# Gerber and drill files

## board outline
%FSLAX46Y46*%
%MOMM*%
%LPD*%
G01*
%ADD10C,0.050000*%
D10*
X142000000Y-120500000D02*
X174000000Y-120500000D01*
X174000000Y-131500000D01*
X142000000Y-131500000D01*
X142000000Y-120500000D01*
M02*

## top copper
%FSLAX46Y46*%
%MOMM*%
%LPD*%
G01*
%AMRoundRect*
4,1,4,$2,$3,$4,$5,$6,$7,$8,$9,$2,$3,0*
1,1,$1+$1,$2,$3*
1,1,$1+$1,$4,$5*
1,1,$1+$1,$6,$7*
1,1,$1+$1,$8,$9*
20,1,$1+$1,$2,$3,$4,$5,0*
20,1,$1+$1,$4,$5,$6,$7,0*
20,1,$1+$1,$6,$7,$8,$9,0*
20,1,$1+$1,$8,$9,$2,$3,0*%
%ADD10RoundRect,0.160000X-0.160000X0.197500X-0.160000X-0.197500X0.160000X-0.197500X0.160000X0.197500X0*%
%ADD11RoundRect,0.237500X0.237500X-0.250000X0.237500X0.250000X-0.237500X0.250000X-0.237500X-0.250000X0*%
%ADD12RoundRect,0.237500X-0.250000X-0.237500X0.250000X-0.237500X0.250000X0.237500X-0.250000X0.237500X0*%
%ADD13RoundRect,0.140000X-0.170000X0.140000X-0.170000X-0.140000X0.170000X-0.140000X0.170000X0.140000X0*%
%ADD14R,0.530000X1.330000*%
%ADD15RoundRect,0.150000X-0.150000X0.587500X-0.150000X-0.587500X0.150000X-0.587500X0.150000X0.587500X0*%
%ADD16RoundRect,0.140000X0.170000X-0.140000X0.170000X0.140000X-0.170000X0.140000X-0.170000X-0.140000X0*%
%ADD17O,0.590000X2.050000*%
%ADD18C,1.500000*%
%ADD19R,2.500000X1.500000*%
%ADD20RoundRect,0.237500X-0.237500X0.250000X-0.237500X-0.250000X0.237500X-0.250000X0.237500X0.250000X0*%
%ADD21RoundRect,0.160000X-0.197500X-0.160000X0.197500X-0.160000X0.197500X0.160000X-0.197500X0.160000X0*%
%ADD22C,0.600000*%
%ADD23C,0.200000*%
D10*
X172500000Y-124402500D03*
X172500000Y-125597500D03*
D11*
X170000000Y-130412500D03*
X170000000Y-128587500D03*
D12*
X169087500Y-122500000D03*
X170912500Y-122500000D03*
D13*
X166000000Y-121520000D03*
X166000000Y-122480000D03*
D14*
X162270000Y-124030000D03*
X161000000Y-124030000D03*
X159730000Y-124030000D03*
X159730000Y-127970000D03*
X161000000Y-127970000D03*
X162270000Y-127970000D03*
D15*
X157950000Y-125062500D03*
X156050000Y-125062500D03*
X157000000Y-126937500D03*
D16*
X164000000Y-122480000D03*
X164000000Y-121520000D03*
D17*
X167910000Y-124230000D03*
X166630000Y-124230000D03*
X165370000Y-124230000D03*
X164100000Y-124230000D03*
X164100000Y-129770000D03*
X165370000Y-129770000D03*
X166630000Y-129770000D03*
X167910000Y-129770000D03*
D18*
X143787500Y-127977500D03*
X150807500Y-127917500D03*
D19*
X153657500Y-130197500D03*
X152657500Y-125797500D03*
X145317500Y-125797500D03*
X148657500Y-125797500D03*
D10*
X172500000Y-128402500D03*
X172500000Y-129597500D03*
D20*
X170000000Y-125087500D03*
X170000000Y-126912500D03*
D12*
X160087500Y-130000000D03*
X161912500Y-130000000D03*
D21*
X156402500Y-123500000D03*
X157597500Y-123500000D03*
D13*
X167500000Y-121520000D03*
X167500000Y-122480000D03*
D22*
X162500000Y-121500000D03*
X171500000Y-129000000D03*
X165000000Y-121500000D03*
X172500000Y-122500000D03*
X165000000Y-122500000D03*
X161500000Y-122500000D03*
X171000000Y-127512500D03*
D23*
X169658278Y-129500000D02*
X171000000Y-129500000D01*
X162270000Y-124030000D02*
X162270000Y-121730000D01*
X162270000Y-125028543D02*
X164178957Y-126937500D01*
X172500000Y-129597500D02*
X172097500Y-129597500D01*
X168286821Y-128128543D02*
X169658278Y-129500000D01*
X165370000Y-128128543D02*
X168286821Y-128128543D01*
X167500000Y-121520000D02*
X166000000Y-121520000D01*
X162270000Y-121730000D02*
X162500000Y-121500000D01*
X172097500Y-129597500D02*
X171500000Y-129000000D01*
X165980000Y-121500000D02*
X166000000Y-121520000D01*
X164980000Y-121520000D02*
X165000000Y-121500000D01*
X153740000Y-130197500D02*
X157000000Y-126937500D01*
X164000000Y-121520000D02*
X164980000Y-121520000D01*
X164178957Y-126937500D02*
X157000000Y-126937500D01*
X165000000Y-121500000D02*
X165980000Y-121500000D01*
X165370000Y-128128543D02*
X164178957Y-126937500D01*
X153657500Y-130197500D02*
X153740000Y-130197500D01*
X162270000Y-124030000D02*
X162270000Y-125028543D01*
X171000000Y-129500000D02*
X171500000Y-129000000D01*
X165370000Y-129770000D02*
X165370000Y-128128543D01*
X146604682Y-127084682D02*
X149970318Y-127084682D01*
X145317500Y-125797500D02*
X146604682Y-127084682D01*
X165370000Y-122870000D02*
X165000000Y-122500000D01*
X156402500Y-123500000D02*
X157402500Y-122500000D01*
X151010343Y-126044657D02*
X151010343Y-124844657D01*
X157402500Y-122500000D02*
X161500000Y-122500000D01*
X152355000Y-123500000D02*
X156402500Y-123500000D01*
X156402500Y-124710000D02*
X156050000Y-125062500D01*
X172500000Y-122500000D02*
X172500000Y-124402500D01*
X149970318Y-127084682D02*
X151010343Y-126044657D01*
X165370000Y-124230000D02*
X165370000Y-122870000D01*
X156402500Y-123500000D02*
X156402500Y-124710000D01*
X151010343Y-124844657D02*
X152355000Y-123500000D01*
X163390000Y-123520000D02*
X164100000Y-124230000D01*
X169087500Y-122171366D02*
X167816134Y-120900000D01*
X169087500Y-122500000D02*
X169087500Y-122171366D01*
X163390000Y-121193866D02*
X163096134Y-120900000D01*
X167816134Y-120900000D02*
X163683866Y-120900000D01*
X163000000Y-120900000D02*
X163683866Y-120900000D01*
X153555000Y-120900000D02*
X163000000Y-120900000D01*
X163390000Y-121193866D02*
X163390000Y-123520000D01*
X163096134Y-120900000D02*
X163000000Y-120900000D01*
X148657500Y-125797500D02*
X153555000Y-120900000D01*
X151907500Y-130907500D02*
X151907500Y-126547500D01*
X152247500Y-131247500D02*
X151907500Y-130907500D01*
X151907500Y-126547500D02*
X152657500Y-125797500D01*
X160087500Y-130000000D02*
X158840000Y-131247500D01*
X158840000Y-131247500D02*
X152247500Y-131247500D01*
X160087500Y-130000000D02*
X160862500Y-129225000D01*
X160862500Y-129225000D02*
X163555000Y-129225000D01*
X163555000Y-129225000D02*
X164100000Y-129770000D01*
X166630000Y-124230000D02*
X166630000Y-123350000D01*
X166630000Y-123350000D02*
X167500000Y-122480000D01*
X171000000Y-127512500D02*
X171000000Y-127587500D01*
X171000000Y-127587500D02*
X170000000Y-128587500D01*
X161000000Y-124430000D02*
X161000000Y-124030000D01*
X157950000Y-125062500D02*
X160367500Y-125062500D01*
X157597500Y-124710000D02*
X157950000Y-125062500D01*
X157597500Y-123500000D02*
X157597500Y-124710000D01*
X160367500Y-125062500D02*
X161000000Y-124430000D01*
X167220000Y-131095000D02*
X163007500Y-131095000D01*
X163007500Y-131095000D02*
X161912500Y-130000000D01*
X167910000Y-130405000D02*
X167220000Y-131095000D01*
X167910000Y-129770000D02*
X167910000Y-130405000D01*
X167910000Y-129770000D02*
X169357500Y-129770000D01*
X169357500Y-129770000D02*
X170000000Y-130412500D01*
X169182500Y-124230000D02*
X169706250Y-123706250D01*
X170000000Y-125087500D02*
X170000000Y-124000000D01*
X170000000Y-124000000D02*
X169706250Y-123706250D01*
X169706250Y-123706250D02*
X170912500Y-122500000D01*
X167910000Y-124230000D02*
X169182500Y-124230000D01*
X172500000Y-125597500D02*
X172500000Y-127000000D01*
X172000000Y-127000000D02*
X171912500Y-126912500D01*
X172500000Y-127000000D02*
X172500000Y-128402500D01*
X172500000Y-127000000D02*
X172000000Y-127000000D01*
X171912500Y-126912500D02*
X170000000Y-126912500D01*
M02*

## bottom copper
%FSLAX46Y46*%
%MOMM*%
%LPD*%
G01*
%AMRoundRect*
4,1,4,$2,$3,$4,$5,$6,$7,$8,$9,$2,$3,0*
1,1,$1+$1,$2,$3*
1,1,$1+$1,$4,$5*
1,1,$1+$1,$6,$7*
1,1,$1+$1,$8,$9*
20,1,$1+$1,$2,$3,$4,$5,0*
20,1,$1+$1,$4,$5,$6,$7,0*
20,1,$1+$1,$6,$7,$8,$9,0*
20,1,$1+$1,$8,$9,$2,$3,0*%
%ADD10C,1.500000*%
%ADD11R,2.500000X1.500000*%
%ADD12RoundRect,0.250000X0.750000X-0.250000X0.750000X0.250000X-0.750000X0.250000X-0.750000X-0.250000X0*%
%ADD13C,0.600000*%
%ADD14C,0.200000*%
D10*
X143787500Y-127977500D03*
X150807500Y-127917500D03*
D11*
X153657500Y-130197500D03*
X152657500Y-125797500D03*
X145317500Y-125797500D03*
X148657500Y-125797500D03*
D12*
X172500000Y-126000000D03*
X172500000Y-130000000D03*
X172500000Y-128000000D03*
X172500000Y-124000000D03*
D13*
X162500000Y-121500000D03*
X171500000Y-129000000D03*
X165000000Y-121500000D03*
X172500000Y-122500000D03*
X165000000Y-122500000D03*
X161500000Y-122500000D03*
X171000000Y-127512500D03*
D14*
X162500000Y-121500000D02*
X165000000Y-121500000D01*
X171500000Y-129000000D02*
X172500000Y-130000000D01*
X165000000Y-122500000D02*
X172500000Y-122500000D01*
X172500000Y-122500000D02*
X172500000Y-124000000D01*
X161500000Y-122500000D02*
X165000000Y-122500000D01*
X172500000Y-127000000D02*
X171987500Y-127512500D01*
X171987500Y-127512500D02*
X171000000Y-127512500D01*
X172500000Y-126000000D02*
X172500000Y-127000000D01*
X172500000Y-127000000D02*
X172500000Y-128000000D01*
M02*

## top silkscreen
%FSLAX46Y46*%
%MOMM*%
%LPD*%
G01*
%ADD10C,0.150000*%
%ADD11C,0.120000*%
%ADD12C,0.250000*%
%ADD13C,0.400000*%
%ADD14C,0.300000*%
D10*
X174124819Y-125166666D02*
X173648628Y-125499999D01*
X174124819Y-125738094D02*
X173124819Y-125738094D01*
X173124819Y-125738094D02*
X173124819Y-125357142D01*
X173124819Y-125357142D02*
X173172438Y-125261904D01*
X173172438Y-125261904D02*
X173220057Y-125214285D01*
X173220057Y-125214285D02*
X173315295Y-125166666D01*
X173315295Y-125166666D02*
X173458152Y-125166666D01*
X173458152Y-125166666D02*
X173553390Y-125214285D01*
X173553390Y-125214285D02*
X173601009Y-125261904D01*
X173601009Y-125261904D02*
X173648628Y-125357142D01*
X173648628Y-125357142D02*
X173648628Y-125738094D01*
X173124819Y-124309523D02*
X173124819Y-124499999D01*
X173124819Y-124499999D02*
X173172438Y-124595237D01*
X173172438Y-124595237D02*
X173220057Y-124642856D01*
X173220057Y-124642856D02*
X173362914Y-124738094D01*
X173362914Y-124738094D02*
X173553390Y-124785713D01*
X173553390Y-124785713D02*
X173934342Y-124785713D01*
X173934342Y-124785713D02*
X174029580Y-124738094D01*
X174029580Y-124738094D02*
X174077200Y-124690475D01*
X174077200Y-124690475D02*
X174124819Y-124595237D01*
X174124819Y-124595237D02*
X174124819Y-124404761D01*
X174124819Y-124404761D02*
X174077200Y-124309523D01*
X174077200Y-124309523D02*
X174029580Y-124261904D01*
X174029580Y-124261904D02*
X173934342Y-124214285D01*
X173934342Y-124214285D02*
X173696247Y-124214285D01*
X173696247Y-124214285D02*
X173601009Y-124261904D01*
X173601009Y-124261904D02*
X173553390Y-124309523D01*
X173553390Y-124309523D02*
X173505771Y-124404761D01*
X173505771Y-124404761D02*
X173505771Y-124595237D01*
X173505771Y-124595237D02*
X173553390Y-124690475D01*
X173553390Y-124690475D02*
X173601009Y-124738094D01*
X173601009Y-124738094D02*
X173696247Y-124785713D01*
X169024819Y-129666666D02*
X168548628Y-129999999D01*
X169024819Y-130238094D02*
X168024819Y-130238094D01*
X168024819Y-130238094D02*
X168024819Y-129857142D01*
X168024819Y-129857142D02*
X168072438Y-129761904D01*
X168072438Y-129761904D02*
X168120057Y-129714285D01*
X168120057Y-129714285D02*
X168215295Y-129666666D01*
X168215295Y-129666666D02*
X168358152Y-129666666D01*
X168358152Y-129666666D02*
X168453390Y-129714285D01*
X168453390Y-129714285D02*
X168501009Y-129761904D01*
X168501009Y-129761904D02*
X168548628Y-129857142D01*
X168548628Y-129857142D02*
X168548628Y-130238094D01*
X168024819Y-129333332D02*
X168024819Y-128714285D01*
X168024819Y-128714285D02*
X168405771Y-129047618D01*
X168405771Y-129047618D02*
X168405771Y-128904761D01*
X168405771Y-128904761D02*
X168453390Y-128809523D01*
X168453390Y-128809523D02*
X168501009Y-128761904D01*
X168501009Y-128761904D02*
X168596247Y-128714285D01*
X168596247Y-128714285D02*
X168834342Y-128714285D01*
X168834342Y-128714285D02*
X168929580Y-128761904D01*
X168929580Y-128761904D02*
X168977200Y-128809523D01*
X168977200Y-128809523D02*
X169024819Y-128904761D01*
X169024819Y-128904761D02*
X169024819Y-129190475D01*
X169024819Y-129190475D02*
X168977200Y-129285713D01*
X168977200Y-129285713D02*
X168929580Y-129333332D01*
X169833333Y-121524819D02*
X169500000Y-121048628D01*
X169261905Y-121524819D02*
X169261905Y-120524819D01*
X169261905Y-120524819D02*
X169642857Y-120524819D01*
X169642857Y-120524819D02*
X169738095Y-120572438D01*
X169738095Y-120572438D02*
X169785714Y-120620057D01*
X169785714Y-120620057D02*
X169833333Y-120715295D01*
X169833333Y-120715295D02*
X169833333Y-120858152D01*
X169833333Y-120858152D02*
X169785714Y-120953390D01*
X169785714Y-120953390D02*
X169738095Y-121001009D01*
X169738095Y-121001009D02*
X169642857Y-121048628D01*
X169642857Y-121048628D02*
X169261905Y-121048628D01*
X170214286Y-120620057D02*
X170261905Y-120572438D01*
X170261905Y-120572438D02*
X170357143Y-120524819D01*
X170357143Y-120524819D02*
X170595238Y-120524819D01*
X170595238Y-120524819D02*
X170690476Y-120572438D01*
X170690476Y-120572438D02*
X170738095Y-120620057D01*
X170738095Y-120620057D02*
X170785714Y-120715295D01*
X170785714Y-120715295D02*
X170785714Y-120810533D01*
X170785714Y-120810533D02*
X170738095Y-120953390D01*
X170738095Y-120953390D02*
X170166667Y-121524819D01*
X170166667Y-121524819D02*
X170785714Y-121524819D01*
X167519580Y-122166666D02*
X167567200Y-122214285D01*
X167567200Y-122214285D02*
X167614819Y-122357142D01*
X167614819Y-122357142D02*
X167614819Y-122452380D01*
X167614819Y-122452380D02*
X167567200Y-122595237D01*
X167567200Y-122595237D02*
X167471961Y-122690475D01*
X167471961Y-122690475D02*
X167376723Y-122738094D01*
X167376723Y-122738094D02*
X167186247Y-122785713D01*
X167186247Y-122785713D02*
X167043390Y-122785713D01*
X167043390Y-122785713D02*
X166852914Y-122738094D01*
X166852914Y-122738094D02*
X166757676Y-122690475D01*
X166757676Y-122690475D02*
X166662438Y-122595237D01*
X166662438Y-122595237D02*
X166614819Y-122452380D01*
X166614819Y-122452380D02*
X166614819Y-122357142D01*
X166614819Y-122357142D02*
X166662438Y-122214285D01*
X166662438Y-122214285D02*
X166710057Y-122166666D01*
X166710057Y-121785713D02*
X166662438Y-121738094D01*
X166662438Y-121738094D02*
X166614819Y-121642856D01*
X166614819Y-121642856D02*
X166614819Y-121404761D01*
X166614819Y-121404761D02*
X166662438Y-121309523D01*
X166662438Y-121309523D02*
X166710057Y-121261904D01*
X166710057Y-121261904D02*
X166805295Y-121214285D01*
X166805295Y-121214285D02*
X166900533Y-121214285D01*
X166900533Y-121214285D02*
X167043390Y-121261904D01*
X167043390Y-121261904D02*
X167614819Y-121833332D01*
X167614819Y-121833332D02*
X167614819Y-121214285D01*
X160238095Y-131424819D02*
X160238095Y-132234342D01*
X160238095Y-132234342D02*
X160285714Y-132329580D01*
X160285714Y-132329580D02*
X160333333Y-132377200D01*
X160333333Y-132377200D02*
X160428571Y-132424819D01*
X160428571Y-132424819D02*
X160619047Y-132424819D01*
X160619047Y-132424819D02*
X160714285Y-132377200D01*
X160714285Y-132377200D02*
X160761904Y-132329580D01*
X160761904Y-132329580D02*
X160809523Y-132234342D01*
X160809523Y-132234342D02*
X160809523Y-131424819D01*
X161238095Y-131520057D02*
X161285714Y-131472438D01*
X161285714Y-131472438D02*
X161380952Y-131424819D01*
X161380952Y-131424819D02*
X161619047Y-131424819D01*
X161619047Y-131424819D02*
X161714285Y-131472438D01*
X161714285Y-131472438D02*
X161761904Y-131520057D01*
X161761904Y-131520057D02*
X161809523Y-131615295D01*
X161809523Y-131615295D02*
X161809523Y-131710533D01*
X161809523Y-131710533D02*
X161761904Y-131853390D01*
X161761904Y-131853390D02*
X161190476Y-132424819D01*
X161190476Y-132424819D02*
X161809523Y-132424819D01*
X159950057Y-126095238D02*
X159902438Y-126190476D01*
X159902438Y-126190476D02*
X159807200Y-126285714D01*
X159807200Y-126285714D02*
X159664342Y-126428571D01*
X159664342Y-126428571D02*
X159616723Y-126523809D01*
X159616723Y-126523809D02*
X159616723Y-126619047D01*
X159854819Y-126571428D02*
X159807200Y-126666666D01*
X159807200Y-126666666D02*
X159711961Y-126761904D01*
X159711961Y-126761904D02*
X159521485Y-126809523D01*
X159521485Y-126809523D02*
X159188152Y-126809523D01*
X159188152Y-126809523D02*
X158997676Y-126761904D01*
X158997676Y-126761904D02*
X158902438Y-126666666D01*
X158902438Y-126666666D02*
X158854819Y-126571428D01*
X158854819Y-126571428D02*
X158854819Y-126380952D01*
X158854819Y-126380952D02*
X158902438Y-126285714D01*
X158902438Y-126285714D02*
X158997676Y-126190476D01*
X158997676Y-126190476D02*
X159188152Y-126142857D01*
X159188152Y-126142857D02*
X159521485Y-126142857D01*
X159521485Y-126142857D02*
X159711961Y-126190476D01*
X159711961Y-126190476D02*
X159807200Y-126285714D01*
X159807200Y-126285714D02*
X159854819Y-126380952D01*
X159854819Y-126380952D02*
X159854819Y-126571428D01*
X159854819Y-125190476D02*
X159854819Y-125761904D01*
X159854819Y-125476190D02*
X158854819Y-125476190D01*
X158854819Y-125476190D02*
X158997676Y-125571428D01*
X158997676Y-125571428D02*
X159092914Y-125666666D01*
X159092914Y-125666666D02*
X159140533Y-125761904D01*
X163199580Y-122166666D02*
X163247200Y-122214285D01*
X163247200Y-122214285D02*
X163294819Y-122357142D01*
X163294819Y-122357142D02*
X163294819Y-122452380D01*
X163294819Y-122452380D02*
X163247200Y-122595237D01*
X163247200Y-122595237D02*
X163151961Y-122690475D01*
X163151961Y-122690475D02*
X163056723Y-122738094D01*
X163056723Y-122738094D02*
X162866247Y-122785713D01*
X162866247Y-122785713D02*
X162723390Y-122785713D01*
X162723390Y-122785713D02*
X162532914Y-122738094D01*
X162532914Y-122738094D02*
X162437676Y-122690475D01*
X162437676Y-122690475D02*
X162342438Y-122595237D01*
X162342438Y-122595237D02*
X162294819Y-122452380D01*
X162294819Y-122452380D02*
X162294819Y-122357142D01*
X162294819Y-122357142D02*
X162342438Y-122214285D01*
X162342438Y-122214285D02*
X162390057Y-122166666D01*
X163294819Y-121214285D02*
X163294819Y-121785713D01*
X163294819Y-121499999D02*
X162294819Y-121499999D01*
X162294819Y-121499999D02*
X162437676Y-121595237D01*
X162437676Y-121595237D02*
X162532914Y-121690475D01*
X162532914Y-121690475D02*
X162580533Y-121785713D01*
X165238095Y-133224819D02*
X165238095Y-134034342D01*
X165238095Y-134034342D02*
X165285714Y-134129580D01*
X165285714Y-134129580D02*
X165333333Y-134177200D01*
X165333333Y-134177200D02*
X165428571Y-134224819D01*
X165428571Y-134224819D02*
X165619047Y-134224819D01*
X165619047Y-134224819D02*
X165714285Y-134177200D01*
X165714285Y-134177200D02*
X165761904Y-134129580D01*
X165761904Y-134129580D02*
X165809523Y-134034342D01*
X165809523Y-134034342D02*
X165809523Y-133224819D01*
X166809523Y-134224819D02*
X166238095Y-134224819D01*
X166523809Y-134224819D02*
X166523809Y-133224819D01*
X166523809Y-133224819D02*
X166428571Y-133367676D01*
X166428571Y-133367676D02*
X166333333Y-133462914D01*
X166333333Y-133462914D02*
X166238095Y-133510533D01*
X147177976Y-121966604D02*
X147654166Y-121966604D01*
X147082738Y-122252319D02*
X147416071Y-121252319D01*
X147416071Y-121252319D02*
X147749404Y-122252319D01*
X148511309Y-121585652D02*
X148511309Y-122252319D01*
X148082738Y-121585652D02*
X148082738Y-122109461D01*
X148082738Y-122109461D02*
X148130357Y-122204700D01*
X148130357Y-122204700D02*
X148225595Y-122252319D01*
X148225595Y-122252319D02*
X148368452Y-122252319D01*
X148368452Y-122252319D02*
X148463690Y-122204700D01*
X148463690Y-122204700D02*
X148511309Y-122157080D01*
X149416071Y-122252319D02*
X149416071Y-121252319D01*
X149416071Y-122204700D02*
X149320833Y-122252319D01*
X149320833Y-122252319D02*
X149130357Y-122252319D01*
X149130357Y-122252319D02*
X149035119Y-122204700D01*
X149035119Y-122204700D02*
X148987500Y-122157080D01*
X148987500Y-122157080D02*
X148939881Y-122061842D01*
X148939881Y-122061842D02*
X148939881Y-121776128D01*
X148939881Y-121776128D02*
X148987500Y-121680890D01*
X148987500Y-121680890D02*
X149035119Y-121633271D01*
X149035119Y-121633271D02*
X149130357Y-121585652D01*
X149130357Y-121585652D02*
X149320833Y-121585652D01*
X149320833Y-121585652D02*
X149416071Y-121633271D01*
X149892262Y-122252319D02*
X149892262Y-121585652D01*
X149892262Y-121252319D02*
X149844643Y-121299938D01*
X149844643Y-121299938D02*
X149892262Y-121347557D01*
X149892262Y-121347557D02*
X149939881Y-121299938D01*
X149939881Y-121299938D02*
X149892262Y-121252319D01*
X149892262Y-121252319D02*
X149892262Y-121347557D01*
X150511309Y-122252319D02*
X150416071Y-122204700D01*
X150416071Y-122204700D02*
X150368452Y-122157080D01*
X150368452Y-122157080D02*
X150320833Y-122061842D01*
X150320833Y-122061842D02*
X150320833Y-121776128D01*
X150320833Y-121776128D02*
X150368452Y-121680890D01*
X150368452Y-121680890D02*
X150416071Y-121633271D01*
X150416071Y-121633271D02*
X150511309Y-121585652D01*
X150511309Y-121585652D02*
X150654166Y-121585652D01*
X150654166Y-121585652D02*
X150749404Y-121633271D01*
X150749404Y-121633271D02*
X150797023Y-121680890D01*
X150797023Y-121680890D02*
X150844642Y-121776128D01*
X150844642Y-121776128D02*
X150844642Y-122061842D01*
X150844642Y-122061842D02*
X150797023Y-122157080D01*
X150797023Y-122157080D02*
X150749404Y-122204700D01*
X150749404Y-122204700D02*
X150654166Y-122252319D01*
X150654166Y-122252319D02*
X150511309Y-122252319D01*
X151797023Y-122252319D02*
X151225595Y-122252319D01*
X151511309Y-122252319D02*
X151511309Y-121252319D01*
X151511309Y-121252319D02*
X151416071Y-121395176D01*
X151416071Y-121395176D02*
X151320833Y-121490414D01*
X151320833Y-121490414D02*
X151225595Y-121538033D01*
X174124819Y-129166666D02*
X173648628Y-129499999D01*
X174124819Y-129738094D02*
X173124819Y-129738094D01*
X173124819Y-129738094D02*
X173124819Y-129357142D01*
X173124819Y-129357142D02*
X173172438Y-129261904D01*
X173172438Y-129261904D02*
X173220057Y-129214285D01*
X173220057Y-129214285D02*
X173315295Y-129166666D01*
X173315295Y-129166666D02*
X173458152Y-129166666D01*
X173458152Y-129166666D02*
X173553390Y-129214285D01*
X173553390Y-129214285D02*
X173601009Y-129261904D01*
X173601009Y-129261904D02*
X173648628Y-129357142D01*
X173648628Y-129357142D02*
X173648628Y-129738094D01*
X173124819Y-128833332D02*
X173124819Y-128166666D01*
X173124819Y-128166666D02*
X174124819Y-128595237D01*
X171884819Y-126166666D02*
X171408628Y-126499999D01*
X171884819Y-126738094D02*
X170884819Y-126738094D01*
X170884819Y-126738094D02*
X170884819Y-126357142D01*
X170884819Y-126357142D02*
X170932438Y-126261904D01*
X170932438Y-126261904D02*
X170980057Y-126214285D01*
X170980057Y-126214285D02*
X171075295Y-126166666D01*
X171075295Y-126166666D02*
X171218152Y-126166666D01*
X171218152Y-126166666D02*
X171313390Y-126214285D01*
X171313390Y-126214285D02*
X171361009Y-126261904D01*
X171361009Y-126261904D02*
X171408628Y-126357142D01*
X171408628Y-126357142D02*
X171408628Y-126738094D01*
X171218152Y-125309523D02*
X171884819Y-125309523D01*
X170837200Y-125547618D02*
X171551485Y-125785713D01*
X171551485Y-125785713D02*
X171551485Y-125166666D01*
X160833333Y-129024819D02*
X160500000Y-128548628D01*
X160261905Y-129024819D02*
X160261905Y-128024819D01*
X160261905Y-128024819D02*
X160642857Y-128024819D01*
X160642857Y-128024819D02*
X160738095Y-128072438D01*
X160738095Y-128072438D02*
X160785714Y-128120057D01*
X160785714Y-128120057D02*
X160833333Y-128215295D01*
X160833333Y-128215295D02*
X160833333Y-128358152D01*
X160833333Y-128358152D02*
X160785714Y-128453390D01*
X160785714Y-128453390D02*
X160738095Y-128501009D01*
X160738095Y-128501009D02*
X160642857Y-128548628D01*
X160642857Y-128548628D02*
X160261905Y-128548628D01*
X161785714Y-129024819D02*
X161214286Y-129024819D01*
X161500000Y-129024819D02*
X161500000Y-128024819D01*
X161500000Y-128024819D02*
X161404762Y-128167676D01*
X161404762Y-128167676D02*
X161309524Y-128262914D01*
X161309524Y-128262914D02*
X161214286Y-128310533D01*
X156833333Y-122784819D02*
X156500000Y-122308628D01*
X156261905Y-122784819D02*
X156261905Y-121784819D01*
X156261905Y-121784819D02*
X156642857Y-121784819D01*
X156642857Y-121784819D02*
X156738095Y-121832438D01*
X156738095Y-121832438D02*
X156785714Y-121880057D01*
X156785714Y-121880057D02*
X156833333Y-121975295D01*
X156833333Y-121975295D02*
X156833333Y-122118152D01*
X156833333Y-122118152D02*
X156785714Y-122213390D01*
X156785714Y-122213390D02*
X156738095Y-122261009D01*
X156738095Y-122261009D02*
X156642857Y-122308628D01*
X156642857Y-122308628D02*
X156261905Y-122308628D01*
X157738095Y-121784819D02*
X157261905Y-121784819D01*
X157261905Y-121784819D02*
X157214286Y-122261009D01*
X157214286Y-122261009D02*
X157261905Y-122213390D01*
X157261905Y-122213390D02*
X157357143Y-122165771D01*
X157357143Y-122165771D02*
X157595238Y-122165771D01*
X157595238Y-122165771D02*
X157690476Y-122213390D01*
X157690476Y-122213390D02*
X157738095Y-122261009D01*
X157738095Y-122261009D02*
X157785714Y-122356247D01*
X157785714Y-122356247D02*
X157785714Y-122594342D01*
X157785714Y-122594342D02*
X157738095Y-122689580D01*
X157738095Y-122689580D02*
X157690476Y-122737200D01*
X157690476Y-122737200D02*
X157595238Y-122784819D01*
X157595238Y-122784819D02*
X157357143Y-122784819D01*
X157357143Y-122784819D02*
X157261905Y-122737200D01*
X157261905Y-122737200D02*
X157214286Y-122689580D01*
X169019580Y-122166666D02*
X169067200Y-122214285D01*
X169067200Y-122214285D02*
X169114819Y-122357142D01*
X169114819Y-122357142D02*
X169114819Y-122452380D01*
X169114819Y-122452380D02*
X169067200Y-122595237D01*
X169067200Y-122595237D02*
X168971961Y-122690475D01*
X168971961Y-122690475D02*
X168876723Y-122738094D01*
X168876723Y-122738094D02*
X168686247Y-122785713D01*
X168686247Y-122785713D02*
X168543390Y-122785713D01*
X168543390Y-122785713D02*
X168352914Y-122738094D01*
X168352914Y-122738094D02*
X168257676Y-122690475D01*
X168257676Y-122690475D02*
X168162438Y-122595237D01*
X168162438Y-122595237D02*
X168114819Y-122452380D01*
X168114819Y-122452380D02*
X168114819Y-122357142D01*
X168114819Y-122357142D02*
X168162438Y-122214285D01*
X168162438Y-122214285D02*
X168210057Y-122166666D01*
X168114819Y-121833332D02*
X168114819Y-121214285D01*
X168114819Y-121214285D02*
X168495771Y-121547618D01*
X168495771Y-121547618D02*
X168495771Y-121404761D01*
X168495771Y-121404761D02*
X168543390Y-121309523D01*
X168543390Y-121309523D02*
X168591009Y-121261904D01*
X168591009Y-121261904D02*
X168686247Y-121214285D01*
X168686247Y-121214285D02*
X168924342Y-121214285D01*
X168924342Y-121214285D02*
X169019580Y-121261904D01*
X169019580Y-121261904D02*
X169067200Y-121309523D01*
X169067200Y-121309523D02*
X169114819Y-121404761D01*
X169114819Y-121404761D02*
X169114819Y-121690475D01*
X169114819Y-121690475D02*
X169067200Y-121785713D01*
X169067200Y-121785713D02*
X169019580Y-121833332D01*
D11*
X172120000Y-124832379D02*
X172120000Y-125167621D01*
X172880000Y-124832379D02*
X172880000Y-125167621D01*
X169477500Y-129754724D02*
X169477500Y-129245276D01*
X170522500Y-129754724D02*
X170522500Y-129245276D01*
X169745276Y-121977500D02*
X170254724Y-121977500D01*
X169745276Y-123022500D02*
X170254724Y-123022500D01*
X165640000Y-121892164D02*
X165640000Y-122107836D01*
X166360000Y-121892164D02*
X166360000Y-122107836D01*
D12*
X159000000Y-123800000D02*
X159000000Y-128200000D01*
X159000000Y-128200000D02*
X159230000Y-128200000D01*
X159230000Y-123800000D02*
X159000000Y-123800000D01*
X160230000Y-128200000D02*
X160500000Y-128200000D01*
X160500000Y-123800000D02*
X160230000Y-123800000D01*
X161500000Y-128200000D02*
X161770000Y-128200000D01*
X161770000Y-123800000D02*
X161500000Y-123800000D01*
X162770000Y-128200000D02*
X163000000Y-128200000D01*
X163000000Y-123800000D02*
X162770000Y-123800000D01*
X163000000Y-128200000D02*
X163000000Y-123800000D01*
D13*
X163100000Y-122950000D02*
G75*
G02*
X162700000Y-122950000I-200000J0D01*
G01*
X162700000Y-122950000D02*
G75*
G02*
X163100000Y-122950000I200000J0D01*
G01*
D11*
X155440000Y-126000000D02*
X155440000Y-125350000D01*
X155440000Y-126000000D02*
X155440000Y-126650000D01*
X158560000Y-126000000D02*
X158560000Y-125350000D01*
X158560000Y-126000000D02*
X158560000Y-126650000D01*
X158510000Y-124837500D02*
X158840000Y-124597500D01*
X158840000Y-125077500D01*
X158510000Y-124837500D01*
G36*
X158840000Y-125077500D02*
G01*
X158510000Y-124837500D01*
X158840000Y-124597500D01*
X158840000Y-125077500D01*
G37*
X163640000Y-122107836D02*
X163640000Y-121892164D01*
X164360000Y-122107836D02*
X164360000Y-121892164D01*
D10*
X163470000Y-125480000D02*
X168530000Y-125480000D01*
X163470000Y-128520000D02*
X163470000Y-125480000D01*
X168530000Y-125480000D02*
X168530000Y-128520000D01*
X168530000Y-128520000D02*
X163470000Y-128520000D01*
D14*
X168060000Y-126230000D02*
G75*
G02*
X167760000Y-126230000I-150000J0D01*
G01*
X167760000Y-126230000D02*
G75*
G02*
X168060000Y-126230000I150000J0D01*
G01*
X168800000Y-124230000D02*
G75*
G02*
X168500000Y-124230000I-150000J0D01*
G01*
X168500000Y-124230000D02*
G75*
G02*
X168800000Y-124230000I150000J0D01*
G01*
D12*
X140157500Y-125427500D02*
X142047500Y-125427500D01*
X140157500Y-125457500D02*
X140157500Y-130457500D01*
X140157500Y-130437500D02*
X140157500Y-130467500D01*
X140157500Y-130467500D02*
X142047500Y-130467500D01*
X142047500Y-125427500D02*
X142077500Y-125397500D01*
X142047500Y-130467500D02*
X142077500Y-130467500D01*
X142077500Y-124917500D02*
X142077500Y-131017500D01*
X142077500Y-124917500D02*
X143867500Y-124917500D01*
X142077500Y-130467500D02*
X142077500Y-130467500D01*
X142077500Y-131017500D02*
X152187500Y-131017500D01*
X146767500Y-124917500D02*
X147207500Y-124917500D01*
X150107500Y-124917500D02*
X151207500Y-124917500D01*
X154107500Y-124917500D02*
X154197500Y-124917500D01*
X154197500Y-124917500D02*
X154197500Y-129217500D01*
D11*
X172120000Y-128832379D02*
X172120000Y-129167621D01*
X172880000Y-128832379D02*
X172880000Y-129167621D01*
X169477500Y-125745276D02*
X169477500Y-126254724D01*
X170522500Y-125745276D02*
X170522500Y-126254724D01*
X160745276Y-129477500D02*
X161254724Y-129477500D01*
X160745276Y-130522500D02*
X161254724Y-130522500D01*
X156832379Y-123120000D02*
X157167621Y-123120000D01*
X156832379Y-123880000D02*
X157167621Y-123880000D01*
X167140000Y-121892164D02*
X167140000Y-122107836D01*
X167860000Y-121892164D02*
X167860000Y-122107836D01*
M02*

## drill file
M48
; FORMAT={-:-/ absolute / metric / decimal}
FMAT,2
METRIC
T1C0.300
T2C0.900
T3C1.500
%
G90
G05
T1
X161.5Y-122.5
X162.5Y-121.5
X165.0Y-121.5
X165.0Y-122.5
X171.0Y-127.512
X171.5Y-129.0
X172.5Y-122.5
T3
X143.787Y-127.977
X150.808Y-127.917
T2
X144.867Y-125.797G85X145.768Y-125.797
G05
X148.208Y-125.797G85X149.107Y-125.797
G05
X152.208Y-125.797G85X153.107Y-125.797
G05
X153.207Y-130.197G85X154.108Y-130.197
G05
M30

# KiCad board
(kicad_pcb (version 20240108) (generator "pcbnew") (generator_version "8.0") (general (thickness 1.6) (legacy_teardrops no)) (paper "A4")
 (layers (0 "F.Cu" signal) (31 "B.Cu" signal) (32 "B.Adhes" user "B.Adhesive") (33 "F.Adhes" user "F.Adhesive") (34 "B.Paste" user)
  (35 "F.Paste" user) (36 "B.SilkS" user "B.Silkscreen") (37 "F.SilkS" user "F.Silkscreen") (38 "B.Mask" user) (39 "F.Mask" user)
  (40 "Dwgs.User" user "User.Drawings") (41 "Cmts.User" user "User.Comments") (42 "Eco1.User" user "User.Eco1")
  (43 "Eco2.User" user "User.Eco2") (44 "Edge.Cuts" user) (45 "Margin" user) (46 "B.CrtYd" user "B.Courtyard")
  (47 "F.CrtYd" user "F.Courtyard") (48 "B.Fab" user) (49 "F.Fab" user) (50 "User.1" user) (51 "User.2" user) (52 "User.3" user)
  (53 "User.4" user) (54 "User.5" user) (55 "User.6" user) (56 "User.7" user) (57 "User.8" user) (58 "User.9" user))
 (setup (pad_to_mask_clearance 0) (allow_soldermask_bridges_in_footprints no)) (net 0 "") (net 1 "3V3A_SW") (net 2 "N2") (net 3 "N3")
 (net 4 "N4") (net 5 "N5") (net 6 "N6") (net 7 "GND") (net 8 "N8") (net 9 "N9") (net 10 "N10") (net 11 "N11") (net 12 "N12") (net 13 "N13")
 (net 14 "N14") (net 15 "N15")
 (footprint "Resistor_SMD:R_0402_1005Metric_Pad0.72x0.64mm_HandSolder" (layer "F.Cu") (at 172.5 125 -90)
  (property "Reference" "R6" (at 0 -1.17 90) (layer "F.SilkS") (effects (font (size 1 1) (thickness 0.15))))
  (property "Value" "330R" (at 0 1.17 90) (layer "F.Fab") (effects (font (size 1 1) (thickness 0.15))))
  (fp_line (start -0.167621 0.38) (end 0.167621 0.38) (stroke (width 0.12) (type solid)) (layer "F.SilkS"))
  (fp_line (start -0.167621 -0.38) (end 0.167621 -0.38) (stroke (width 0.12) (type solid)) (layer "F.SilkS"))
  (pad "1" smd roundrect (at -0.5975 0 270) (size 0.715 0.64) (layers "F.Cu" "F.Paste" "F.Mask") (roundrect_rratio 0.25) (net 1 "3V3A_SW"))
  (pad "2" smd roundrect (at 0.5975 0 270) (size 0.715 0.64) (layers "F.Cu" "F.Paste" "F.Mask") (roundrect_rratio 0.25) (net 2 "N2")))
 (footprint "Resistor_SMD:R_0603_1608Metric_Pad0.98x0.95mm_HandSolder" (layer "F.Cu") (at 170 129.5 90)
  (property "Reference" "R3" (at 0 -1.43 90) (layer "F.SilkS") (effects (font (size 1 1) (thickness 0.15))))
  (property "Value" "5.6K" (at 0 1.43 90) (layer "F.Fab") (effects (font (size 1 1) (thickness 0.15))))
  (fp_line (start -0.254724 -0.5225) (end 0.254724 -0.5225) (stroke (width 0.12) (type solid)) (layer "F.SilkS"))
  (fp_line (start -0.254724 0.5225) (end 0.254724 0.5225) (stroke (width 0.12) (type solid)) (layer "F.SilkS"))
  (pad "1" smd roundrect (at -0.9125 0 90) (size 0.975 0.95) (layers "F.Cu" "F.Paste" "F.Mask") (roundrect_rratio 0.25) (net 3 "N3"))
  (pad "2" smd roundrect (at 0.9125 0 90) (size 0.975 0.95) (layers "F.Cu" "F.Paste" "F.Mask") (roundrect_rratio 0.25) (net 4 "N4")))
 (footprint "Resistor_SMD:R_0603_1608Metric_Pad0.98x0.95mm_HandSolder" (layer "F.Cu") (at 170 122.5)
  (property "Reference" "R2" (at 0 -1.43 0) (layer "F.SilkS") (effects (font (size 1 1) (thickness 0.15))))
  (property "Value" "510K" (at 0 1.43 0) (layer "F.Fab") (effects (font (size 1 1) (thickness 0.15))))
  (fp_line (start -0.254724 -0.5225) (end 0.254724 -0.5225) (stroke (width 0.12) (type solid)) (layer "F.SilkS"))
  (fp_line (start -0.254724 0.5225) (end 0.254724 0.5225) (stroke (width 0.12) (type solid)) (layer "F.SilkS"))
  (pad "1" smd roundrect (at -0.9125 0) (size 0.975 0.95) (layers "F.Cu" "F.Paste" "F.Mask") (roundrect_rratio 0.25) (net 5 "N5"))
  (pad "2" smd roundrect (at 0.9125 0) (size 0.975 0.95) (layers "F.Cu" "F.Paste" "F.Mask") (roundrect_rratio 0.25) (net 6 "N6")))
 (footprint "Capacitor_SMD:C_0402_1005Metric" (layer "F.Cu") (at 166 122 -90)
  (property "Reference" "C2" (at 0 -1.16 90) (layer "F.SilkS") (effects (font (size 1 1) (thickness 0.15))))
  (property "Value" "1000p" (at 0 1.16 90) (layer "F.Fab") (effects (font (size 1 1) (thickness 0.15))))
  (fp_line (start -0.107836 0.36) (end 0.107836 0.36) (stroke (width 0.12) (type solid)) (layer "F.SilkS"))
  (fp_line (start -0.107836 -0.36) (end 0.107836 -0.36) (stroke (width 0.12) (type solid)) (layer "F.SilkS"))
  (pad "1" smd roundrect (at -0.48 0 270) (size 0.56 0.62) (layers "F.Cu" "F.Paste" "F.Mask") (roundrect_rratio 0.25) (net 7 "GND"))
  (pad "2" smd roundrect (at 0.48 0 270) (size 0.56 0.62) (layers "F.Cu" "F.Paste" "F.Mask") (roundrect_rratio 0.25) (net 1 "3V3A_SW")))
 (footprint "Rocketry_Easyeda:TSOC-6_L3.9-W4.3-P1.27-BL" (layer "F.Cu") (at 161 126 180)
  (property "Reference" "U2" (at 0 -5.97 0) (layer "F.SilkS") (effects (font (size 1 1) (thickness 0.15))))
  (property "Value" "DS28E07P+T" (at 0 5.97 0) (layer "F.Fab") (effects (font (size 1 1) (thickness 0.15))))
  (fp_line (start 2 2.2) (end 2 -2.2) (stroke (width 0.25) (type solid)) (layer "F.SilkS"))
  (fp_line (start 2 -2.2) (end 1.77 -2.2) (stroke (width 0.25) (type solid)) (layer "F.SilkS"))
  (fp_line (start 1.77 2.2) (end 2 2.2) (stroke (width 0.25) (type solid)) (layer "F.SilkS"))
  (fp_line (start 0.77 -2.2) (end 0.5 -2.2) (stroke (width 0.25) (type solid)) (layer "F.SilkS"))
  (fp_line (start 0.5 2.2) (end 0.77 2.2) (stroke (width 0.25) (type solid)) (layer "F.SilkS"))
  (fp_line (start -0.5 -2.2) (end -0.77 -2.2) (stroke (width 0.25) (type solid)) (layer "F.SilkS"))
  (fp_line (start -0.77 2.2) (end -0.5 2.2) (stroke (width 0.25) (type solid)) (layer "F.SilkS"))
  (fp_line (start -1.77 -2.2) (end -2 -2.2) (stroke (width 0.25) (type solid)) (layer "F.SilkS"))
  (fp_line (start -2 2.2) (end -1.77 2.2) (stroke (width 0.25) (type solid)) (layer "F.SilkS"))
  (fp_line (start -2 -2.2) (end -2 2.2) (stroke (width 0.25) (type solid)) (layer "F.SilkS"))
  (fp_circle (center -1.9 3.05) (end -1.7 3.05) (stroke (width 0.4) (type solid)) (fill none) (layer "F.SilkS"))
  (pad "1" smd rect (at -1.27 1.97 180) (size 0.53 1.33) (layers "F.Cu" "F.Paste" "F.Mask") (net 7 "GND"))
  (pad "2" smd rect (at 0 1.97 180) (size 0.53 1.33) (layers "F.Cu" "F.Paste" "F.Mask") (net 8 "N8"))
  (pad "3" smd rect (at 1.27 1.97 180) (size 0.53 1.33) (layers "F.Cu" "F.Paste" "F.Mask") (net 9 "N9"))
  (pad "4" smd rect (at 1.27 -1.97 180) (size 0.53 1.33) (layers "F.Cu" "F.Paste" "F.Mask") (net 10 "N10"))
  (pad "5" smd rect (at 0 -1.97 180) (size 0.53 1.33) (layers "F.Cu" "F.Paste" "F.Mask") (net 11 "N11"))
  (pad "6" smd rect (at -1.27 -1.97 180) (size 0.53 1.33) (layers "F.Cu" "F.Paste" "F.Mask") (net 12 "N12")))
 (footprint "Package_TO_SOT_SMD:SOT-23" (layer "F.Cu") (at 157 126 -90)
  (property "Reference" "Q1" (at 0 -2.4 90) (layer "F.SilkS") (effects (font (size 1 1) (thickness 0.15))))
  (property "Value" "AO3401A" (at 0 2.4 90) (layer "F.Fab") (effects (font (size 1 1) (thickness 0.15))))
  (fp_line (start 0 1.56) (end -0.65 1.56) (stroke (width 0.12) (type solid)) (layer "F.SilkS"))
  (fp_line (start 0 1.56) (end 0.65 1.56) (stroke (width 0.12) (type solid)) (layer "F.SilkS"))
  (fp_line (start 0 -1.56) (end -0.65 -1.56) (stroke (width 0.12) (type solid)) (layer "F.SilkS"))
  (fp_line (start 0 -1.56) (end 0.65 -1.56) (stroke (width 0.12) (type solid)) (layer "F.SilkS"))
  (fp_poly
   (pts (xy -1.1625 -1.51) (xy -1.4025 -1.84) (xy -0.9225 -1.84) (xy -1.1625 -1.51)) (stroke (width 0.12) (type solid)) (fill solid)
   (layer "F.SilkS"))
  (pad "1" smd roundrect (at -0.9375 -0.95 270) (size 1.475 0.6) (layers "F.Cu" "F.Paste" "F.Mask") (roundrect_rratio 0.25) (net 8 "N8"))
  (pad "2" smd roundrect (at -0.9375 0.95 270) (size 1.475 0.6) (layers "F.Cu" "F.Paste" "F.Mask") (roundrect_rratio 0.25) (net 1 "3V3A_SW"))
  (pad "3" smd roundrect (at 0.9375 0 270) (size 1.475 0.6) (layers "F.Cu" "F.Paste" "F.Mask") (roundrect_rratio 0.25) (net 7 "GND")))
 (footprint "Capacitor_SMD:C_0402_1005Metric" (layer "F.Cu") (at 164 122 90)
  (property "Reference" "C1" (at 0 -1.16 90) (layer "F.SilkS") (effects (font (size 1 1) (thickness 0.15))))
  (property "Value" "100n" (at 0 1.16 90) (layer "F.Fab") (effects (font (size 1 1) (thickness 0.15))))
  (fp_line (start -0.107836 -0.36) (end 0.107836 -0.36) (stroke (width 0.12) (type solid)) (layer "F.SilkS"))
  (fp_line (start -0.107836 0.36) (end 0.107836 0.36) (stroke (width 0.12) (type solid)) (layer "F.SilkS"))
  (pad "1" smd roundrect (at -0.48 0 90) (size 0.56 0.62) (layers "F.Cu" "F.Paste" "F.Mask") (roundrect_rratio 0.25) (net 1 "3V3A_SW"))
  (pad "2" smd roundrect (at 0.48 0 90) (size 0.56 0.62) (layers "F.Cu" "F.Paste" "F.Mask") (roundrect_rratio 0.25) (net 7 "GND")))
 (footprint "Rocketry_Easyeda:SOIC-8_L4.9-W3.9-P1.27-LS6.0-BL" (layer "F.Cu") (at 166 127 180)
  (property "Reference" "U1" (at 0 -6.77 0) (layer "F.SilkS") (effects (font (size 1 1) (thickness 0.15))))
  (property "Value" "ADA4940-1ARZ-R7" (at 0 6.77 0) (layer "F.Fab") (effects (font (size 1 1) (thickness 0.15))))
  (fp_line (start 2.53 1.52) (end -2.53 1.52) (stroke (width 0.15) (type solid)) (layer "F.SilkS"))
  (fp_line (start 2.53 -1.52) (end 2.53 1.52) (stroke (width 0.15) (type solid)) (layer "F.SilkS"))
  (fp_line (start -2.53 1.52) (end -2.53 -1.52) (stroke (width 0.15) (type solid)) (layer "F.SilkS"))
  (fp_line (start -2.53 -1.52) (end 2.53 -1.52) (stroke (width 0.15) (type solid)) (layer "F.SilkS"))
  (fp_circle (center -1.91 0.77) (end -1.76 0.77) (stroke (width 0.3) (type solid)) (fill none) (layer "F.SilkS"))
  (fp_circle (center -2.65 2.77) (end -2.5 2.77) (stroke (width 0.3) (type solid)) (fill none) (layer "F.SilkS"))
  (pad "1" smd oval (at -1.91 2.77 180) (size 0.59 2.05) (layers "F.Cu" "F.Paste" "F.Mask") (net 6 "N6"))
  (pad "2" smd oval (at -0.63 2.77 180) (size 0.59 2.05) (layers "F.Cu" "F.Paste" "F.Mask") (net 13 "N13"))
  (pad "3" smd oval (at 0.63 2.77 180) (size 0.59 2.05) (layers "F.Cu" "F.Paste" "F.Mask") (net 1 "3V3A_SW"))
  (pad "4" smd oval (at 1.9 2.77 180) (size 0.59 2.05) (layers "F.Cu" "F.Paste" "F.Mask") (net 5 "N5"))
  (pad "5" smd oval (at 1.9 -2.77 180) (size 0.59 2.05) (layers "F.Cu" "F.Paste" "F.Mask") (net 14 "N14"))
  (pad "6" smd oval (at 0.63 -2.77 180) (size 0.59 2.05) (layers "F.Cu" "F.Paste" "F.Mask") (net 7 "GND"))
  (pad "7" smd oval (at -0.63 -2.77 180) (size 0.59 2.05) (layers "F.Cu" "F.Paste" "F.Mask") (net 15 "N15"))
  (pad "8" smd oval (at -1.91 -2.77 180) (size 0.59 2.05) (layers "F.Cu" "F.Paste" "F.Mask") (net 3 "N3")))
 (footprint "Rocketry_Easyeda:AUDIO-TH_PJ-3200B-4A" (layer "F.Cu") (at 149.4875 127.9975)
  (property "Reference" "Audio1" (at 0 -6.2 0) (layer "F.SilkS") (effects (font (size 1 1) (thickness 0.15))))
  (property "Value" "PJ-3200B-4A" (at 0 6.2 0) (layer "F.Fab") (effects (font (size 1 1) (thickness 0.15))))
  (fp_line (start -9.33 -2.57) (end -7.44 -2.57) (stroke (width 0.25) (type solid)) (layer "F.SilkS"))
  (fp_line (start -9.33 -2.54) (end -9.33 2.46) (stroke (width 0.25) (type solid)) (layer "F.SilkS"))
  (fp_line (start -9.33 2.44) (end -9.33 2.47) (stroke (width 0.25) (type solid)) (layer "F.SilkS"))
  (fp_line (start -9.33 2.47) (end -7.44 2.47) (stroke (width 0.25) (type solid)) (layer "F.SilkS"))
  (fp_line (start -7.44 -2.57) (end -7.41 -2.6) (stroke (width 0.25) (type solid)) (layer "F.SilkS"))
  (fp_line (start -7.44 2.47) (end -7.41 2.47) (stroke (width 0.25) (type solid)) (layer "F.SilkS"))
  (fp_line (start -7.41 -3.08) (end -7.41 3.02) (stroke (width 0.25) (type solid)) (layer "F.SilkS"))
  (fp_line (start -7.41 -3.08) (end -5.62 -3.08) (stroke (width 0.25) (type solid)) (layer "F.SilkS"))
  (fp_line (start -7.41 2.47) (end -7.41 2.47) (stroke (width 0.25) (type solid)) (layer "F.SilkS"))
  (fp_line (start -7.41 3.02) (end 2.7 3.02) (stroke (width 0.25) (type solid)) (layer "F.SilkS"))
  (fp_line (start -2.72 -3.08) (end -2.28 -3.08) (stroke (width 0.25) (type solid)) (layer "F.SilkS"))
  (fp_line (start 0.62 -3.08) (end 1.72 -3.08) (stroke (width 0.25) (type solid)) (layer "F.SilkS"))
  (fp_line (start 4.62 -3.08) (end 4.71 -3.08) (stroke (width 0.25) (type solid)) (layer "F.SilkS"))
  (fp_line (start 4.71 -3.08) (end 4.71 1.22) (stroke (width 0.25) (type solid)) (layer "F.SilkS"))
  (pad "" thru_hole circle (at -5.7 -0.02) (size 1.5 1.5) (drill 1.5) (layers "*.Cu" "*.Mask") (remove_unused_layers no))
  (pad "" thru_hole circle (at 1.32 -0.08) (size 1.5 1.5) (drill 1.5) (layers "*.Cu" "*.Mask") (remove_unused_layers no))
  (pad "1" thru_hole rect (at 4.17 2.2 90) (size 1.5 2.5) (drill oval 0.900024 1.8002) (layers "*.Cu" "*.Mask") (remove_unused_layers no)
   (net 7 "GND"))
  (pad "2" thru_hole rect (at 3.17 -2.2 90) (size 1.5 2.5) (drill oval 0.900024 1.799946) (layers "*.Cu" "*.Mask") (remove_unused_layers no)
   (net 14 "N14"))
  (pad "3" thru_hole rect (at -4.17 -2.2 90) (size 1.5 2.5) (drill oval 0.900024 1.8002) (layers "*.Cu" "*.Mask") (remove_unused_layers no)
   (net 1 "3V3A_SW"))
  (pad "4" thru_hole rect (at -0.83 -2.2 90) (size 1.5 2.5) (drill oval 0.900024 1.799946) (layers "*.Cu" "*.Mask")
   (remove_unused_layers no) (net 5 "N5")))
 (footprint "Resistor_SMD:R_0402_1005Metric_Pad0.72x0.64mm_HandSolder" (layer "F.Cu") (at 172.5 129 -90)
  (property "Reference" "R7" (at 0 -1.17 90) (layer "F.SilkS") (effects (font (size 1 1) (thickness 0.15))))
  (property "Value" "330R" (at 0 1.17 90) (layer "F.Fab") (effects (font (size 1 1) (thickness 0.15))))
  (fp_line (start -0.167621 0.38) (end 0.167621 0.38) (stroke (width 0.12) (type solid)) (layer "F.SilkS"))
  (fp_line (start -0.167621 -0.38) (end 0.167621 -0.38) (stroke (width 0.12) (type solid)) (layer "F.SilkS"))
  (pad "1" smd roundrect (at -0.5975 0 270) (size 0.715 0.64) (layers "F.Cu" "F.Paste" "F.Mask") (roundrect_rratio 0.25) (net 2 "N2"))
  (pad "2" smd roundrect (at 0.5975 0 270) (size 0.715 0.64) (layers "F.Cu" "F.Paste" "F.Mask") (roundrect_rratio 0.25) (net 7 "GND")))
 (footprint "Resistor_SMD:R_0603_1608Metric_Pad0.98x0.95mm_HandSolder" (layer "F.Cu") (at 170 126 -90)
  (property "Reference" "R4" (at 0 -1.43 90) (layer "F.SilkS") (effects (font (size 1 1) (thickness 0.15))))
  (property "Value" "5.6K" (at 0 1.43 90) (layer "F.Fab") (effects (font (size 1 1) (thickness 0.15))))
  (fp_line (start -0.254724 0.5225) (end 0.254724 0.5225) (stroke (width 0.12) (type solid)) (layer "F.SilkS"))
  (fp_line (start -0.254724 -0.5225) (end 0.254724 -0.5225) (stroke (width 0.12) (type solid)) (layer "F.SilkS"))
  (pad "1" smd roundrect (at -0.9125 0 270) (size 0.975 0.95) (layers "F.Cu" "F.Paste" "F.Mask") (roundrect_rratio 0.25) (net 6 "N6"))
  (pad "2" smd roundrect (at 0.9125 0 270) (size 0.975 0.95) (layers "F.Cu" "F.Paste" "F.Mask") (roundrect_rratio 0.25) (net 2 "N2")))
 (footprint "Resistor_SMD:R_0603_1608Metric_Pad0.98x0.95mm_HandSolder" (layer "F.Cu") (at 161 130)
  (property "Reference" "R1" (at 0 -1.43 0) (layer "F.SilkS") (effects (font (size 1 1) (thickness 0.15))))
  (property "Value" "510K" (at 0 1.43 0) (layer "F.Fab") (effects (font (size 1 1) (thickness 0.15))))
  (fp_line (start -0.254724 -0.5225) (end 0.254724 -0.5225) (stroke (width 0.12) (type solid)) (layer "F.SilkS"))
  (fp_line (start -0.254724 0.5225) (end 0.254724 0.5225) (stroke (width 0.12) (type solid)) (layer "F.SilkS"))
  (pad "1" smd roundrect (at -0.9125 0) (size 0.975 0.95) (layers "F.Cu" "F.Paste" "F.Mask") (roundrect_rratio 0.25) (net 14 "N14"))
  (pad "2" smd roundrect (at 0.9125 0) (size 0.975 0.95) (layers "F.Cu" "F.Paste" "F.Mask") (roundrect_rratio 0.25) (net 3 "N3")))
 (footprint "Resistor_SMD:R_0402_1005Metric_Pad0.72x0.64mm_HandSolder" (layer "F.Cu") (at 157 123.5)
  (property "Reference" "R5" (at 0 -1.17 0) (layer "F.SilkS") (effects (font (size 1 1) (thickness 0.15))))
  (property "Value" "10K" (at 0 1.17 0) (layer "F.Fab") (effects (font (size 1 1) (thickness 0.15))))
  (fp_line (start -0.167621 -0.38) (end 0.167621 -0.38) (stroke (width 0.12) (type solid)) (layer "F.SilkS"))
  (fp_line (start -0.167621 0.38) (end 0.167621 0.38) (stroke (width 0.12) (type solid)) (layer "F.SilkS"))
  (pad "1" smd roundrect (at -0.5975 0) (size 0.715 0.64) (layers "F.Cu" "F.Paste" "F.Mask") (roundrect_rratio 0.25) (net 1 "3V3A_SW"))
  (pad "2" smd roundrect (at 0.5975 0) (size 0.715 0.64) (layers "F.Cu" "F.Paste" "F.Mask") (roundrect_rratio 0.25) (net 8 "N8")))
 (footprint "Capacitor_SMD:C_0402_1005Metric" (layer "F.Cu") (at 167.5 122 -90)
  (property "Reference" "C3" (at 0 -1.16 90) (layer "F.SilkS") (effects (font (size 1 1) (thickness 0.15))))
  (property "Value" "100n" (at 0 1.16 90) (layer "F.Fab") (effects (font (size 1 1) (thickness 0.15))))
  (fp_line (start -0.107836 0.36) (end 0.107836 0.36) (stroke (width 0.12) (type solid)) (layer "F.SilkS"))
  (fp_line (start -0.107836 -0.36) (end 0.107836 -0.36) (stroke (width 0.12) (type solid)) (layer "F.SilkS"))
  (pad "1" smd roundrect (at -0.48 0 270) (size 0.56 0.62) (layers "F.Cu" "F.Paste" "F.Mask") (roundrect_rratio 0.25) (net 7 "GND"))
  (pad "2" smd roundrect (at 0.48 0 270) (size 0.56 0.62) (layers "F.Cu" "F.Paste" "F.Mask") (roundrect_rratio 0.25) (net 13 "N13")))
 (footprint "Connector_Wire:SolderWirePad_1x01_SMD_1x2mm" (layer "B.Cu") (at 172.5 126 90)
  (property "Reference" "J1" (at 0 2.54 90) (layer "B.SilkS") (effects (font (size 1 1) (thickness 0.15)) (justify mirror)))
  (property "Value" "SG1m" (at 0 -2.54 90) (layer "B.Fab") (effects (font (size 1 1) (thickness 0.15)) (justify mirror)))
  (pad "1" smd roundrect (at 0 0 90) (size 1 2) (layers "B.Cu" "B.Paste" "B.Mask") (roundrect_rratio 0.25) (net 4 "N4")))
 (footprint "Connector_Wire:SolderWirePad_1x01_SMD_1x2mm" (layer "B.Cu") (at 172.5 130 90)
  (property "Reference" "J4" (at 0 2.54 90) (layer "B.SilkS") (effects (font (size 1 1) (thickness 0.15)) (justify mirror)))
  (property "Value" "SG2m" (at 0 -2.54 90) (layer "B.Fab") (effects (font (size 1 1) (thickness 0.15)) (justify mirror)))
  (pad "1" smd roundrect (at 0 0 90) (size 1 2) (layers "B.Cu" "B.Paste" "B.Mask") (roundrect_rratio 0.25) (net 7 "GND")))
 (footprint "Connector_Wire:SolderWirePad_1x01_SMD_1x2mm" (layer "B.Cu") (at 172.5 128 90)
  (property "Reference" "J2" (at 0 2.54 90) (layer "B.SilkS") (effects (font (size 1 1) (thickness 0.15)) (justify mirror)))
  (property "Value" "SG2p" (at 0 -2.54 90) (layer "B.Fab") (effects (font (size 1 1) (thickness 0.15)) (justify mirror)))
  (pad "1" smd roundrect (at 0 0 90) (size 1 2) (layers "B.Cu" "B.Paste" "B.Mask") (roundrect_rratio 0.25) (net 4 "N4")))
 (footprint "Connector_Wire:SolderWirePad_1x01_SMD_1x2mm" (layer "B.Cu") (at 172.5 124 90)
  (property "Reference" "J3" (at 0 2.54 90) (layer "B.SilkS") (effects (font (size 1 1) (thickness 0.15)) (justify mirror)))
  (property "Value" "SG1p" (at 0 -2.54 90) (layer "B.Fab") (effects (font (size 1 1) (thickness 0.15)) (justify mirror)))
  (pad "1" smd roundrect (at 0 0 90) (size 1 2) (layers "B.Cu" "B.Paste" "B.Mask") (roundrect_rratio 0.25) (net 1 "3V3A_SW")))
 (gr_rect (start 142 120.5) (end 174 131.5) (stroke (width 0.05) (type default)) (fill none) (layer "Edge.Cuts"))
 (segment (start 169.658278 129.5) (end 171 129.5) (width 0.2) (layer "F.Cu") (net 7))
 (segment (start 162.27 124.03) (end 162.27 121.73) (width 0.2) (layer "F.Cu") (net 7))
 (segment (start 162.27 125.028543) (end 164.178957 126.9375) (width 0.2) (layer "F.Cu") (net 7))
 (segment (start 172.5 129.5975) (end 172.0975 129.5975) (width 0.2) (layer "F.Cu") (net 7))
 (segment (start 168.286821 128.128543) (end 169.658278 129.5) (width 0.2) (layer "F.Cu") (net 7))
 (segment (start 165.37 128.128543) (end 168.286821 128.128543) (width 0.2) (layer "F.Cu") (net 7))
 (segment (start 167.5 121.52) (end 166 121.52) (width 0.2) (layer "F.Cu") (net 7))
 (segment (start 162.27 121.73) (end 162.5 121.5) (width 0.2) (layer "F.Cu") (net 7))
 (segment (start 172.0975 129.5975) (end 171.5 129) (width 0.2) (layer "F.Cu") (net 7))
 (segment (start 165.98 121.5) (end 166 121.52) (width 0.2) (layer "F.Cu") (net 7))
 (segment (start 164.98 121.52) (end 165 121.5) (width 0.2) (layer "F.Cu") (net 7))
 (segment (start 153.74 130.1975) (end 157 126.9375) (width 0.2) (layer "F.Cu") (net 7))
 (segment (start 164 121.52) (end 164.98 121.52) (width 0.2) (layer "F.Cu") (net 7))
 (segment (start 164.178957 126.9375) (end 157 126.9375) (width 0.2) (layer "F.Cu") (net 7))
 (segment (start 165 121.5) (end 165.98 121.5) (width 0.2) (layer "F.Cu") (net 7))
 (segment (start 165.37 128.128543) (end 164.178957 126.9375) (width 0.2) (layer "F.Cu") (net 7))
 (segment (start 153.6575 130.1975) (end 153.74 130.1975) (width 0.2) (layer "F.Cu") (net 7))
 (segment (start 162.27 124.03) (end 162.27 125.028543) (width 0.2) (layer "F.Cu") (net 7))
 (segment (start 171 129.5) (end 171.5 129) (width 0.2) (layer "F.Cu") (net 7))
 (segment (start 165.37 129.77) (end 165.37 128.128543) (width 0.2) (layer "F.Cu") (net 7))
 (via (at 162.5 121.5) (size 0.6) (drill 0.3) (layers "F.Cu" "B.Cu") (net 7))
 (via (at 171.5 129) (size 0.6) (drill 0.3) (layers "F.Cu" "B.Cu") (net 7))
 (via (at 165 121.5) (size 0.6) (drill 0.3) (layers "F.Cu" "B.Cu") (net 7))
 (segment (start 162.5 121.5) (end 165 121.5) (width 0.2) (layer "B.Cu") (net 7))
 (segment (start 171.5 129) (end 172.5 130) (width 0.2) (layer "B.Cu") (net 7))
 (segment (start 146.604682 127.084682) (end 149.970318 127.084682) (width 0.2) (layer "F.Cu") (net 1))
 (segment (start 145.3175 125.7975) (end 146.604682 127.084682) (width 0.2) (layer "F.Cu") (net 1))
 (segment (start 165.37 122.87) (end 165 122.5) (width 0.2) (layer "F.Cu") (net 1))
 (segment (start 156.4025 123.5) (end 157.4025 122.5) (width 0.2) (layer "F.Cu") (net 1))
 (segment (start 151.010343 126.044657) (end 151.010343 124.844657) (width 0.2) (layer "F.Cu") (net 1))
 (segment (start 157.4025 122.5) (end 161.5 122.5) (width 0.2) (layer "F.Cu") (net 1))
 (segment (start 152.355 123.5) (end 156.4025 123.5) (width 0.2) (layer "F.Cu") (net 1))
 (segment (start 156.4025 124.71) (end 156.05 125.0625) (width 0.2) (layer "F.Cu") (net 1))
 (segment (start 172.5 122.5) (end 172.5 124.4025) (width 0.2) (layer "F.Cu") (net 1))
 (segment (start 149.970318 127.084682) (end 151.010343 126.044657) (width 0.2) (layer "F.Cu") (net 1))
 (segment (start 165.37 124.23) (end 165.37 122.87) (width 0.2) (layer "F.Cu") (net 1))
 (segment (start 156.4025 123.5) (end 156.4025 124.71) (width 0.2) (layer "F.Cu") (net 1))
 (segment (start 151.010343 124.844657) (end 152.355 123.5) (width 0.2) (layer "F.Cu") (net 1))
 (via (at 172.5 122.5) (size 0.6) (drill 0.3) (layers "F.Cu" "B.Cu") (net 1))
 (via (at 165 122.5) (size 0.6) (drill 0.3) (layers "F.Cu" "B.Cu") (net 1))
 (via (at 161.5 122.5) (size 0.6) (drill 0.3) (layers "F.Cu" "B.Cu") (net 1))
 (segment (start 165 122.5) (end 172.5 122.5) (width 0.2) (layer "B.Cu") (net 1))
 (segment (start 172.5 122.5) (end 172.5 124) (width 0.2) (layer "B.Cu") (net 1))
 (segment (start 161.5 122.5) (end 165 122.5) (width 0.2) (layer "B.Cu") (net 1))
 (segment (start 163.39 123.52) (end 164.1 124.23) (width 0.2) (layer "F.Cu") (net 5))
 (segment (start 169.0875 122.171366) (end 167.816134 120.9) (width 0.2) (layer "F.Cu") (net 5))
 (segment (start 169.0875 122.5) (end 169.0875 122.171366) (width 0.2) (layer "F.Cu") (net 5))
 (segment (start 163.39 121.193866) (end 163.096134 120.9) (width 0.2) (layer "F.Cu") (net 5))
 (segment (start 167.816134 120.9) (end 163.683866 120.9) (width 0.2) (layer "F.Cu") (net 5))
 (segment (start 163 120.9) (end 163.683866 120.9) (width 0.2) (layer "F.Cu") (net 5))
 (segment (start 153.555 120.9) (end 163 120.9) (width 0.2) (layer "F.Cu") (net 5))
 (segment (start 163.39 121.193866) (end 163.39 123.52) (width 0.2) (layer "F.Cu") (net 5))
 (segment (start 163.096134 120.9) (end 163 120.9) (width 0.2) (layer "F.Cu") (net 5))
 (segment (start 148.6575 125.7975) (end 153.555 120.9) (width 0.2) (layer "F.Cu") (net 5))
 (segment (start 151.9075 130.9075) (end 151.9075 126.5475) (width 0.2) (layer "F.Cu") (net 14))
 (segment (start 152.2475 131.2475) (end 151.9075 130.9075) (width 0.2) (layer "F.Cu") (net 14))
 (segment (start 151.9075 126.5475) (end 152.6575 125.7975) (width 0.2) (layer "F.Cu") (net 14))
 (segment (start 160.0875 130) (end 158.84 131.2475) (width 0.2) (layer "F.Cu") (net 14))
 (segment (start 158.84 131.2475) (end 152.2475 131.2475) (width 0.2) (layer "F.Cu") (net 14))
 (segment (start 160.0875 130) (end 160.8625 129.225) (width 0.2) (layer "F.Cu") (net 14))
 (segment (start 160.8625 129.225) (end 163.555 129.225) (width 0.2) (layer "F.Cu") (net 14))
 (segment (start 163.555 129.225) (end 164.1 129.77) (width 0.2) (layer "F.Cu") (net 14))
 (segment (start 166.63 124.23) (end 166.63 123.35) (width 0.2) (layer "F.Cu") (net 13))
 (segment (start 166.63 123.35) (end 167.5 122.48) (width 0.2) (layer "F.Cu") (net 13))
 (segment (start 171 127.5125) (end 171 127.5875) (width 0.2) (layer "F.Cu") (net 4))
 (segment (start 171 127.5875) (end 170 128.5875) (width 0.2) (layer "F.Cu") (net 4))
 (via (at 171 127.5125) (size 0.6) (drill 0.3) (layers "F.Cu" "B.Cu") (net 4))
 (segment (start 172.5 127) (end 171.9875 127.5125) (width 0.2) (layer "B.Cu") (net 4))
 (segment (start 171.9875 127.5125) (end 171 127.5125) (width 0.2) (layer "B.Cu") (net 4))
 (segment (start 172.5 126) (end 172.5 127) (width 0.2) (layer "B.Cu") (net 4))
 (segment (start 172.5 127) (end 172.5 128) (width 0.2) (layer "B.Cu") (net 4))
 (segment (start 161 124.43) (end 161 124.03) (width 0.2) (layer "F.Cu") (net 8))
 (segment (start 157.95 125.0625) (end 160.3675 125.0625) (width 0.2) (layer "F.Cu") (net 8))
 (segment (start 157.5975 124.71) (end 157.95 125.0625) (width 0.2) (layer "F.Cu") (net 8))
 (segment (start 157.5975 123.5) (end 157.5975 124.71) (width 0.2) (layer "F.Cu") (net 8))
 (segment (start 160.3675 125.0625) (end 161 124.43) (width 0.2) (layer "F.Cu") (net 8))
 (segment (start 167.22 131.095) (end 163.0075 131.095) (width 0.2) (layer "F.Cu") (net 3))
 (segment (start 163.0075 131.095) (end 161.9125 130) (width 0.2) (layer "F.Cu") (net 3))
 (segment (start 167.91 130.405) (end 167.22 131.095) (width 0.2) (layer "F.Cu") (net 3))
 (segment (start 167.91 129.77) (end 167.91 130.405) (width 0.2) (layer "F.Cu") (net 3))
 (segment (start 167.91 129.77) (end 169.3575 129.77) (width 0.2) (layer "F.Cu") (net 3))
 (segment (start 169.3575 129.77) (end 170 130.4125) (width 0.2) (layer "F.Cu") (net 3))
 (segment (start 169.1825 124.23) (end 169.70625 123.70625) (width 0.2) (layer "F.Cu") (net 6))
 (segment (start 170 125.0875) (end 170 124) (width 0.2) (layer "F.Cu") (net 6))
 (segment (start 170 124) (end 169.70625 123.70625) (width 0.2) (layer "F.Cu") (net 6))
 (segment (start 169.70625 123.70625) (end 170.9125 122.5) (width 0.2) (layer "F.Cu") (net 6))
 (segment (start 167.91 124.23) (end 169.1825 124.23) (width 0.2) (layer "F.Cu") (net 6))
 (segment (start 172.5 125.5975) (end 172.5 127) (width 0.2) (layer "F.Cu") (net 2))
 (segment (start 172 127) (end 171.9125 126.9125) (width 0.2) (layer "F.Cu") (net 2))
 (segment (start 172.5 127) (end 172.5 128.4025) (width 0.2) (layer "F.Cu") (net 2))
 (segment (start 172.5 127) (end 172 127) (width 0.2) (layer "F.Cu") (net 2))
 (segment (start 171.9125 126.9125) (end 170 126.9125) (width 0.2) (layer "F.Cu") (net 2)))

